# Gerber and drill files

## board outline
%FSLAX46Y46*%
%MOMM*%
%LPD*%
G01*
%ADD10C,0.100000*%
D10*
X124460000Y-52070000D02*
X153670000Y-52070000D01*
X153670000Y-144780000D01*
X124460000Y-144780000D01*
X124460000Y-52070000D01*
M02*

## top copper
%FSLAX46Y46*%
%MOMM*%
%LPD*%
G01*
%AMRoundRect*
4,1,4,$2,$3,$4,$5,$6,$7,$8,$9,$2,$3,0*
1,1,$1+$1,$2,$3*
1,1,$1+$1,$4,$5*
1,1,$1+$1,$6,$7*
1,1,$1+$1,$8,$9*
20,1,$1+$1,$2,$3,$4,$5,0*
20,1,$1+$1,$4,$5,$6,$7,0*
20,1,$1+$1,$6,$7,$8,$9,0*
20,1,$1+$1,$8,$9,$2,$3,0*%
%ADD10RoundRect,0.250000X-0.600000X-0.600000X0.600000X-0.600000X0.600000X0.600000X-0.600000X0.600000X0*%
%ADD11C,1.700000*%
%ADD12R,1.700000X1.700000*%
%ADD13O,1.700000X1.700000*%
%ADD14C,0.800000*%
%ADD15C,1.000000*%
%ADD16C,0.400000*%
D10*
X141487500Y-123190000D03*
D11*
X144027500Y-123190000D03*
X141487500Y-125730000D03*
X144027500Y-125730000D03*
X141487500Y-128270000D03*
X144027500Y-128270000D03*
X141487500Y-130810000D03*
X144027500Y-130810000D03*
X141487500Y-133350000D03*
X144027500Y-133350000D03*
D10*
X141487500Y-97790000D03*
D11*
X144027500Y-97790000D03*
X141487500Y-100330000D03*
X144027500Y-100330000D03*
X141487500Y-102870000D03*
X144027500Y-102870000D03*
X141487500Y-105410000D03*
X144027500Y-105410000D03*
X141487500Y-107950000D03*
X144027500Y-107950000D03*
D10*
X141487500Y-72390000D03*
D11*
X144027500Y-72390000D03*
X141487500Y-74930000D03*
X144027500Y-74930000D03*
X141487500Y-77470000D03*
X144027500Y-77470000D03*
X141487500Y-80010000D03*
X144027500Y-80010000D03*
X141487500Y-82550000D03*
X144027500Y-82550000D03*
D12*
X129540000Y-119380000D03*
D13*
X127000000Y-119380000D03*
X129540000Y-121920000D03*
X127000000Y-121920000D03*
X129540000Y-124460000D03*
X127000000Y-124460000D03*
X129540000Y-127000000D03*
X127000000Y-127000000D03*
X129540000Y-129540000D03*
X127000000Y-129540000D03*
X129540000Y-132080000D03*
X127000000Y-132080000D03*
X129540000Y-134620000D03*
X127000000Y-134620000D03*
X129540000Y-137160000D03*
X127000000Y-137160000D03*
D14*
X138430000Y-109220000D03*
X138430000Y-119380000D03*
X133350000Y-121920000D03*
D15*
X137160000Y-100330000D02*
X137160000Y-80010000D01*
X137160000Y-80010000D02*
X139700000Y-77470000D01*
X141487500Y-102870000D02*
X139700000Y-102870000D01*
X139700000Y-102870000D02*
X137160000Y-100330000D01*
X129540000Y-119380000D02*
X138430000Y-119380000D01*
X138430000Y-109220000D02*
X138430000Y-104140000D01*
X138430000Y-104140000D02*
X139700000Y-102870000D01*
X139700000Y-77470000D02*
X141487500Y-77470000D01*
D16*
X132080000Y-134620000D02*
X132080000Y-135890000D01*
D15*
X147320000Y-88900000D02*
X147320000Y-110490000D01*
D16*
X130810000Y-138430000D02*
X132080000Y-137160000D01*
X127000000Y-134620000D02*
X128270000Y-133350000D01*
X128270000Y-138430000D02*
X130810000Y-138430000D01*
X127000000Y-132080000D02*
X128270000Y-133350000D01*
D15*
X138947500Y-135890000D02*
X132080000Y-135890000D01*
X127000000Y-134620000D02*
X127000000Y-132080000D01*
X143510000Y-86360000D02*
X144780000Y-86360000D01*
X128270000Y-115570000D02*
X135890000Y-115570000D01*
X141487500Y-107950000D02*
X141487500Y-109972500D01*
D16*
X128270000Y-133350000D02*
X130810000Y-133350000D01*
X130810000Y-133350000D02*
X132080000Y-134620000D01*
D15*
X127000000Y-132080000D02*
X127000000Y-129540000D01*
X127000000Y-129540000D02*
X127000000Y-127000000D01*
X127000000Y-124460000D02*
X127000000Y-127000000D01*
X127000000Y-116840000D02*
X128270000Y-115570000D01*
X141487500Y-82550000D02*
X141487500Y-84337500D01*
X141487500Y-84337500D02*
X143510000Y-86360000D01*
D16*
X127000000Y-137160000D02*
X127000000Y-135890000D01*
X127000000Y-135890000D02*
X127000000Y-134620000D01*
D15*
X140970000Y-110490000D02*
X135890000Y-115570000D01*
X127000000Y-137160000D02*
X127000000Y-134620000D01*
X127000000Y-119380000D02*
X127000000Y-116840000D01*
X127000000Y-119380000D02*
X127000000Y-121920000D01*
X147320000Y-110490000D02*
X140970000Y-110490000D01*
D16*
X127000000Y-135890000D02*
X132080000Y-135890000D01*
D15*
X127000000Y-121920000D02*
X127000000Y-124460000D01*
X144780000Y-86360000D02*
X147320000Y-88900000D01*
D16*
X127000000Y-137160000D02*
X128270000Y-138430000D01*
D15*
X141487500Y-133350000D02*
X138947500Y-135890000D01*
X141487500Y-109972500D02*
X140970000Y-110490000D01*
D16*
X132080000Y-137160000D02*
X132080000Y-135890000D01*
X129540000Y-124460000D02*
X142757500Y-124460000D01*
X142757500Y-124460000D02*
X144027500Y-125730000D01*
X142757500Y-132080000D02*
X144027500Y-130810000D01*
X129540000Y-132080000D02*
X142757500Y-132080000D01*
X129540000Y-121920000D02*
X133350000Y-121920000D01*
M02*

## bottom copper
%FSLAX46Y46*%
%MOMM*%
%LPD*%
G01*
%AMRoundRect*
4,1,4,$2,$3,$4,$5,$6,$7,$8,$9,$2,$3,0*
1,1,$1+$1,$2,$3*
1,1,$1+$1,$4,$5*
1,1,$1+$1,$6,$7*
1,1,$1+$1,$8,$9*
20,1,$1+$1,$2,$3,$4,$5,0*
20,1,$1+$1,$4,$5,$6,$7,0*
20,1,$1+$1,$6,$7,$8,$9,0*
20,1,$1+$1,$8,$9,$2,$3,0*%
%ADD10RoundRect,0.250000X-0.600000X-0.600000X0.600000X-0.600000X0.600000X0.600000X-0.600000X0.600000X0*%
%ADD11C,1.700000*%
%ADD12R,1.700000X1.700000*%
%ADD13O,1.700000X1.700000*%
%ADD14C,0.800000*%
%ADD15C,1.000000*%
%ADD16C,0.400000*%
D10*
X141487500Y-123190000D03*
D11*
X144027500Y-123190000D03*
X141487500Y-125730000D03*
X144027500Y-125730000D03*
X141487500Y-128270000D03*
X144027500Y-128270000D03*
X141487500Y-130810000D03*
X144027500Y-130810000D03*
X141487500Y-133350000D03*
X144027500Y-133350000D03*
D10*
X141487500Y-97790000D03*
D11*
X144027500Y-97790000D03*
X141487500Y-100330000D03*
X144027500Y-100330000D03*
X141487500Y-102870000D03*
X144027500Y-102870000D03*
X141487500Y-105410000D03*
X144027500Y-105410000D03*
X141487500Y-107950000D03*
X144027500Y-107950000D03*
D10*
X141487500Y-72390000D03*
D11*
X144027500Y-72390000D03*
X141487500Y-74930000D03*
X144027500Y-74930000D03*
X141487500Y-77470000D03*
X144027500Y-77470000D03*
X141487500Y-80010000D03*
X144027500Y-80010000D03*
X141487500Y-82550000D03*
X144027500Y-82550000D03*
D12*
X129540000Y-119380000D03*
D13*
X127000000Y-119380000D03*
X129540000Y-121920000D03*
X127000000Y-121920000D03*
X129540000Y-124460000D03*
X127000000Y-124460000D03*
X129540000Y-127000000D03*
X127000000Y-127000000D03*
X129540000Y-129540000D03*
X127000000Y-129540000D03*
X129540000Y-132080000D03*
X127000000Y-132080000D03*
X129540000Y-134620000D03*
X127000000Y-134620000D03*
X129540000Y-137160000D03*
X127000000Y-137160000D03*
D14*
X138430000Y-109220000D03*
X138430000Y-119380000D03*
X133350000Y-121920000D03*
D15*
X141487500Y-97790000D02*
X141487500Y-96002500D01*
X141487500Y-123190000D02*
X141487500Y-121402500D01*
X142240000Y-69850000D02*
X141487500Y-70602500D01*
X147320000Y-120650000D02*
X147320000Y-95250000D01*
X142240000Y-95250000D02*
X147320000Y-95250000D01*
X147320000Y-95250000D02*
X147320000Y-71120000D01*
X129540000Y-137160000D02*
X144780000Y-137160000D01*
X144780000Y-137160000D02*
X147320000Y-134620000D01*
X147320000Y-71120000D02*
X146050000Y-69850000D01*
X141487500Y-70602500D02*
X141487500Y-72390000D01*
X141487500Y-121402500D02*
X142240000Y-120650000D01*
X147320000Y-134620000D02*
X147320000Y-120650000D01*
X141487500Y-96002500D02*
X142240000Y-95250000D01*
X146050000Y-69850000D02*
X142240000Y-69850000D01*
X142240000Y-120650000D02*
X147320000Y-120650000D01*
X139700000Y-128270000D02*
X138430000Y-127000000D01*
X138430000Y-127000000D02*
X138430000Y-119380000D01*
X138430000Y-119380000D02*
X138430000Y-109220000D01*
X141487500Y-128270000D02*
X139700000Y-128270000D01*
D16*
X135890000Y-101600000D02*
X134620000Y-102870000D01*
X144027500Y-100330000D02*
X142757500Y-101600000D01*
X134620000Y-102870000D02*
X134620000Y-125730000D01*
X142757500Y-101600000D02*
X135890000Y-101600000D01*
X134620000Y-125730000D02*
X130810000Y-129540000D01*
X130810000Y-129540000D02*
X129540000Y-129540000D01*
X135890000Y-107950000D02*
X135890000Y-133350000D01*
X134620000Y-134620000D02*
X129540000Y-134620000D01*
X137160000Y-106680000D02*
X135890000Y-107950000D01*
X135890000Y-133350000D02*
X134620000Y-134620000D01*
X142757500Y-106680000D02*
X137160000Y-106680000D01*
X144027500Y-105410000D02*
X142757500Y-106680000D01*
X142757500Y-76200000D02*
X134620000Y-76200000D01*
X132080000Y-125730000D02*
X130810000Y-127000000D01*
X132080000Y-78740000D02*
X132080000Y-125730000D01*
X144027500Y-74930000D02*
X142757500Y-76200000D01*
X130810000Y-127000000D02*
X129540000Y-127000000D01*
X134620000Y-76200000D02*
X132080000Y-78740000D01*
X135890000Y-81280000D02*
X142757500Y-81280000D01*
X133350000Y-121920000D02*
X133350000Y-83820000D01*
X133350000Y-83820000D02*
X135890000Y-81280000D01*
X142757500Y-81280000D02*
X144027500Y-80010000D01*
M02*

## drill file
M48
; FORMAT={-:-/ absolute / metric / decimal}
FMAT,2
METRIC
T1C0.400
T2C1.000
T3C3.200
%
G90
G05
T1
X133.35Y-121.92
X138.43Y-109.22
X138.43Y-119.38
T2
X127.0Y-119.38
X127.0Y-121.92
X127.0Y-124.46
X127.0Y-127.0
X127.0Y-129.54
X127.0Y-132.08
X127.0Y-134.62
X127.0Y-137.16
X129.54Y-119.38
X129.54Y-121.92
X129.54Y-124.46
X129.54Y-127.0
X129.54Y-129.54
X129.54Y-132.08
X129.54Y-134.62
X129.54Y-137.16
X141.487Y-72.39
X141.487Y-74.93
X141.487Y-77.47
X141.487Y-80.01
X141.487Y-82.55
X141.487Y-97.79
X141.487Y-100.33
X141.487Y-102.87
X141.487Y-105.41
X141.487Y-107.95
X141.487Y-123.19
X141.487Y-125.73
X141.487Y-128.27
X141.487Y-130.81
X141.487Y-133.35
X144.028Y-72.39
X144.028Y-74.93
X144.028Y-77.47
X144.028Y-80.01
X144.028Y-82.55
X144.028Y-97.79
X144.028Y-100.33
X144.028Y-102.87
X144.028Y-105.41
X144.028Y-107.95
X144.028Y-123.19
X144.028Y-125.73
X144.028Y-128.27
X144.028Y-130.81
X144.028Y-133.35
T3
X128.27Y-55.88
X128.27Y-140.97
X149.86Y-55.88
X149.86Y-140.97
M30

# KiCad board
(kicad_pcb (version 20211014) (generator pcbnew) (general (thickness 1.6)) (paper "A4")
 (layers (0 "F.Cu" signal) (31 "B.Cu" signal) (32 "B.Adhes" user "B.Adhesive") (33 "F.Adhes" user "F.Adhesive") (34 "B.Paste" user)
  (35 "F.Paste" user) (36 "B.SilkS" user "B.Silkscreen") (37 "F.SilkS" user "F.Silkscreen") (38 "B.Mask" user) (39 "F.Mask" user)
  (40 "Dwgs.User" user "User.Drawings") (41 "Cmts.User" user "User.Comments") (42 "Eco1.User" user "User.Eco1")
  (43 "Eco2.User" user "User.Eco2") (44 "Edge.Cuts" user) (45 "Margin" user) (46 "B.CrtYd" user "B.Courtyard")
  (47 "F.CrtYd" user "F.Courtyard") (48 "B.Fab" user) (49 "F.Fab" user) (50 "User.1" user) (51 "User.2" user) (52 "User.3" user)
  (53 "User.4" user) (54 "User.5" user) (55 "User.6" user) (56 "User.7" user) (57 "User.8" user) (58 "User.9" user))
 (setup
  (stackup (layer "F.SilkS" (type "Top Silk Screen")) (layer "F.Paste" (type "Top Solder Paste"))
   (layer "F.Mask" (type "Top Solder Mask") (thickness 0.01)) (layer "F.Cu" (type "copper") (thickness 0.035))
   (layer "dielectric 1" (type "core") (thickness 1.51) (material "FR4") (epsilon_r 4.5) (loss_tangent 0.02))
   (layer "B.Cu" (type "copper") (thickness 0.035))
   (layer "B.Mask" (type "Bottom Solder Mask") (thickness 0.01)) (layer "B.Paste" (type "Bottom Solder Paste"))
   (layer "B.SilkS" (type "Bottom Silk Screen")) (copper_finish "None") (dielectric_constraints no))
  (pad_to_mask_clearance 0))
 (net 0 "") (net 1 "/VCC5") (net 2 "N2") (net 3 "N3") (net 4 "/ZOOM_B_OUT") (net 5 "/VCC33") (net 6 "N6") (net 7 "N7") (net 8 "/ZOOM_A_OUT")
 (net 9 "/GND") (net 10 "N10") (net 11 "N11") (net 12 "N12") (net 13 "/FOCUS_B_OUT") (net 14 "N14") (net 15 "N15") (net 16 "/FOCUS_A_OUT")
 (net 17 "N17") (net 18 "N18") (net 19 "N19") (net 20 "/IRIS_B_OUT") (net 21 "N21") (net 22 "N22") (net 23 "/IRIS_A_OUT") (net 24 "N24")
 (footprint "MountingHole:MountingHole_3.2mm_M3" (layer "F.Cu") (at 149.86 55.88)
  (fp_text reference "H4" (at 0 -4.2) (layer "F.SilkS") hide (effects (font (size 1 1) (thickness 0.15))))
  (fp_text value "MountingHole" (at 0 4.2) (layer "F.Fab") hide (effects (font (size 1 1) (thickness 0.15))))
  (pad "" np_thru_hole circle locked (at 0 0) (size 3.2 3.2) (drill 3.2) (layers *.Cu *.Mask)))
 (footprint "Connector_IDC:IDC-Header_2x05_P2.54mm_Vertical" (layer "F.Cu") (at 141.4875 123.19)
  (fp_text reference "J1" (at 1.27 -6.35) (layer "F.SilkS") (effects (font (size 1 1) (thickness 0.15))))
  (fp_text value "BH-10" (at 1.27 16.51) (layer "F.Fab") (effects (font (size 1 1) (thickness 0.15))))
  (pad "1" thru_hole roundrect locked (at 0 0) (size 1.7 1.7) (drill 1) (layers *.Cu *.Mask) (roundrect_rratio 0.1470588235) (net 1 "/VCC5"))
  (pad "2" thru_hole circle locked (at 2.54 0) (size 1.7 1.7) (drill 1) (layers *.Cu *.Mask) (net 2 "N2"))
  (pad "3" thru_hole circle locked (at 0 2.54) (size 1.7 1.7) (drill 1) (layers *.Cu *.Mask) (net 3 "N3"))
  (pad "4" thru_hole circle locked (at 2.54 2.54) (size 1.7 1.7) (drill 1) (layers *.Cu *.Mask) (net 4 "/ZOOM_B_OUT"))
  (pad "5" thru_hole circle locked (at 0 5.08) (size 1.7 1.7) (drill 1) (layers *.Cu *.Mask) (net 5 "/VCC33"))
  (pad "6" thru_hole circle locked (at 2.54 5.08) (size 1.7 1.7) (drill 1) (layers *.Cu *.Mask) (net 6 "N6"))
  (pad "7" thru_hole circle locked (at 0 7.62) (size 1.7 1.7) (drill 1) (layers *.Cu *.Mask) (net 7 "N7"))
  (pad "8" thru_hole circle locked (at 2.54 7.62) (size 1.7 1.7) (drill 1) (layers *.Cu *.Mask) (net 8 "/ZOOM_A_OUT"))
  (pad "9" thru_hole circle locked (at 0 10.16) (size 1.7 1.7) (drill 1) (layers *.Cu *.Mask) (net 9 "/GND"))
  (pad "10" thru_hole circle locked (at 2.54 10.16) (size 1.7 1.7) (drill 1) (layers *.Cu *.Mask) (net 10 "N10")))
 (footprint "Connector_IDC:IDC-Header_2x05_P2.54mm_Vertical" (layer "F.Cu") (at 141.4875 97.79)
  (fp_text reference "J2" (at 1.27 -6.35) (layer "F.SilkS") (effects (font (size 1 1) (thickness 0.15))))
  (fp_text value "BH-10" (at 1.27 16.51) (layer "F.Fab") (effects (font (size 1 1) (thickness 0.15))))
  (pad "1" thru_hole roundrect locked (at 0 0) (size 1.7 1.7) (drill 1) (layers *.Cu *.Mask) (roundrect_rratio 0.1470588235) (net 1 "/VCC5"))
  (pad "2" thru_hole circle locked (at 2.54 0) (size 1.7 1.7) (drill 1) (layers *.Cu *.Mask) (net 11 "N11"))
  (pad "3" thru_hole circle locked (at 0 2.54) (size 1.7 1.7) (drill 1) (layers *.Cu *.Mask) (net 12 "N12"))
  (pad "4" thru_hole circle locked (at 2.54 2.54) (size 1.7 1.7) (drill 1) (layers *.Cu *.Mask) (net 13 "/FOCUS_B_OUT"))
  (pad "5" thru_hole circle locked (at 0 5.08) (size 1.7 1.7) (drill 1) (layers *.Cu *.Mask) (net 5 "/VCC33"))
  (pad "6" thru_hole circle locked (at 2.54 5.08) (size 1.7 1.7) (drill 1) (layers *.Cu *.Mask) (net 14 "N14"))
  (pad "7" thru_hole circle locked (at 0 7.62) (size 1.7 1.7) (drill 1) (layers *.Cu *.Mask) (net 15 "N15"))
  (pad "8" thru_hole circle locked (at 2.54 7.62) (size 1.7 1.7) (drill 1) (layers *.Cu *.Mask) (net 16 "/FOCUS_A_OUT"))
  (pad "9" thru_hole circle locked (at 0 10.16) (size 1.7 1.7) (drill 1) (layers *.Cu *.Mask) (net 9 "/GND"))
  (pad "10" thru_hole circle locked (at 2.54 10.16) (size 1.7 1.7) (drill 1) (layers *.Cu *.Mask) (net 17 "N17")))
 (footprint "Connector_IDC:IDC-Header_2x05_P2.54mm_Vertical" (layer "F.Cu") (at 141.4875 72.39)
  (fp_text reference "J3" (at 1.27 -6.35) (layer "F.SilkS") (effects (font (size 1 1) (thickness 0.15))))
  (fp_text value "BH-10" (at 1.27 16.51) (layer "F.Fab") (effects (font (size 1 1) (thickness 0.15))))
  (pad "1" thru_hole roundrect locked (at 0 0) (size 1.7 1.7) (drill 1) (layers *.Cu *.Mask) (roundrect_rratio 0.1470588235) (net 1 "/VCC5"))
  (pad "2" thru_hole circle locked (at 2.54 0) (size 1.7 1.7) (drill 1) (layers *.Cu *.Mask) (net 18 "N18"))
  (pad "3" thru_hole circle locked (at 0 2.54) (size 1.7 1.7) (drill 1) (layers *.Cu *.Mask) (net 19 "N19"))
  (pad "4" thru_hole circle locked (at 2.54 2.54) (size 1.7 1.7) (drill 1) (layers *.Cu *.Mask) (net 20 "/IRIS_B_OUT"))
  (pad "5" thru_hole circle locked (at 0 5.08) (size 1.7 1.7) (drill 1) (layers *.Cu *.Mask) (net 5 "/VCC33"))
  (pad "6" thru_hole circle locked (at 2.54 5.08) (size 1.7 1.7) (drill 1) (layers *.Cu *.Mask) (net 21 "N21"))
  (pad "7" thru_hole circle locked (at 0 7.62) (size 1.7 1.7) (drill 1) (layers *.Cu *.Mask) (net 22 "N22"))
  (pad "8" thru_hole circle locked (at 2.54 7.62) (size 1.7 1.7) (drill 1) (layers *.Cu *.Mask) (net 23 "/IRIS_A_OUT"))
  (pad "9" thru_hole circle locked (at 0 10.16) (size 1.7 1.7) (drill 1) (layers *.Cu *.Mask) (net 9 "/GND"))
  (pad "10" thru_hole circle locked (at 2.54 10.16) (size 1.7 1.7) (drill 1) (layers *.Cu *.Mask) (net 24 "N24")))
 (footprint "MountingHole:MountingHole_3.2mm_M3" (layer "F.Cu") (at 128.27 140.97)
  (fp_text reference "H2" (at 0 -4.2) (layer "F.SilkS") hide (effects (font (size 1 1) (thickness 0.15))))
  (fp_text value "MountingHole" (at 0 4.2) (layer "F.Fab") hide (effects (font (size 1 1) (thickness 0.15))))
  (pad "" np_thru_hole circle locked (at 0 0) (size 3.2 3.2) (drill 3.2) (layers *.Cu *.Mask)))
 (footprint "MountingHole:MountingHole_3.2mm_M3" (layer "F.Cu") (at 149.86 140.97)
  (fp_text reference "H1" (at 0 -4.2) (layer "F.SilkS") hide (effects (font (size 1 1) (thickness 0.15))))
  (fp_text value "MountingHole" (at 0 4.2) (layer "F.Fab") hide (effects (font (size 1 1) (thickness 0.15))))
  (pad "" np_thru_hole circle locked (at 0 0) (size 3.2 3.2) (drill 3.2) (layers *.Cu *.Mask)))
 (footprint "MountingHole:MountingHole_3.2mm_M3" (layer "F.Cu") (at 128.27 55.88)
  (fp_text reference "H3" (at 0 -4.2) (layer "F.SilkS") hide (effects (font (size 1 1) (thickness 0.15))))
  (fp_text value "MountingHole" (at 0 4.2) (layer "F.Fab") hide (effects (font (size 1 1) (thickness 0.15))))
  (pad "" np_thru_hole circle locked (at 0 0) (size 3.2 3.2) (drill 3.2) (layers *.Cu *.Mask)))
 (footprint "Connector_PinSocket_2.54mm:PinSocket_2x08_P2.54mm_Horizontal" (layer "F.Cu") (at 129.54 119.38)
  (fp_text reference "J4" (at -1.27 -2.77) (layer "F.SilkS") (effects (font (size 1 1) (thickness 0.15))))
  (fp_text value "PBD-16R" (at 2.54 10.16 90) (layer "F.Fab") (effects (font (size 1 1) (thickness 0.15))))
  (pad "1" thru_hole rect locked (at 0 0) (size 1.7 1.7) (drill 1) (layers *.Cu *.Mask) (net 5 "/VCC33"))
  (pad "2" thru_hole oval locked (at -2.54 0) (size 1.7 1.7) (drill 1) (layers *.Cu *.Mask) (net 9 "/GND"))
  (pad "3" thru_hole oval locked (at 0 2.54) (size 1.7 1.7) (drill 1) (layers *.Cu *.Mask) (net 23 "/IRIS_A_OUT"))
  (pad "4" thru_hole oval locked (at -2.54 2.54) (size 1.7 1.7) (drill 1) (layers *.Cu *.Mask) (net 9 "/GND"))
  (pad "5" thru_hole oval locked (at 0 5.08) (size 1.7 1.7) (drill 1) (layers *.Cu *.Mask) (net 4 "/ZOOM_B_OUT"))
  (pad "6" thru_hole oval locked (at -2.54 5.08) (size 1.7 1.7) (drill 1) (layers *.Cu *.Mask) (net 9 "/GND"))
  (pad "7" thru_hole oval locked (at 0 7.62) (size 1.7 1.7) (drill 1) (layers *.Cu *.Mask) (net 20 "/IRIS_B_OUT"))
  (pad "8" thru_hole oval locked (at -2.54 7.62) (size 1.7 1.7) (drill 1) (layers *.Cu *.Mask) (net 9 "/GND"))
  (pad "9" thru_hole oval locked (at 0 10.16) (size 1.7 1.7) (drill 1) (layers *.Cu *.Mask) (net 13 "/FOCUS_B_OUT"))
  (pad "10" thru_hole oval locked (at -2.54 10.16) (size 1.7 1.7) (drill 1) (layers *.Cu *.Mask) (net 9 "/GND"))
  (pad "11" thru_hole oval locked (at 0 12.7) (size 1.7 1.7) (drill 1) (layers *.Cu *.Mask) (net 8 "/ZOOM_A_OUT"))
  (pad "12" thru_hole oval locked (at -2.54 12.7) (size 1.7 1.7) (drill 1) (layers *.Cu *.Mask) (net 9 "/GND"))
  (pad "13" thru_hole oval locked (at 0 15.24) (size 1.7 1.7) (drill 1) (layers *.Cu *.Mask) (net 16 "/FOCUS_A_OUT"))
  (pad "14" thru_hole oval locked (at -2.54 15.24) (size 1.7 1.7) (drill 1) (layers *.Cu *.Mask) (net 9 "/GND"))
  (pad "15" thru_hole oval locked (at 0 17.78) (size 1.7 1.7) (drill 1) (layers *.Cu *.Mask) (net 1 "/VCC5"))
  (pad "16" thru_hole oval locked (at -2.54 17.78) (size 1.7 1.7) (drill 1) (layers *.Cu *.Mask) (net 9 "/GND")))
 (gr_rect (start 124.46 52.07) (end 153.67 144.78) (layer "Edge.Cuts") (width 0.1) (fill none))
 (segment (start 141.4875 97.79) (end 141.4875 96.0025) (width 1) (layer "B.Cu") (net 1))
 (segment (start 141.4875 123.19) (end 141.4875 121.4025) (width 1) (layer "B.Cu") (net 1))
 (segment (start 142.24 69.85) (end 141.4875 70.6025) (width 1) (layer "B.Cu") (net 1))
 (segment (start 147.32 120.65) (end 147.32 95.25) (width 1) (layer "B.Cu") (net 1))
 (segment (start 142.24 95.25) (end 147.32 95.25) (width 1) (layer "B.Cu") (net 1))
 (segment (start 147.32 95.25) (end 147.32 71.12) (width 1) (layer "B.Cu") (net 1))
 (segment (start 129.54 137.16) (end 144.78 137.16) (width 1) (layer "B.Cu") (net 1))
 (segment (start 144.78 137.16) (end 147.32 134.62) (width 1) (layer "B.Cu") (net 1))
 (segment (start 147.32 71.12) (end 146.05 69.85) (width 1) (layer "B.Cu") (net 1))
 (segment (start 141.4875 70.6025) (end 141.4875 72.39) (width 1) (layer "B.Cu") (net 1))
 (segment (start 141.4875 121.4025) (end 142.24 120.65) (width 1) (layer "B.Cu") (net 1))
 (segment (start 147.32 134.62) (end 147.32 120.65) (width 1) (layer "B.Cu") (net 1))
 (segment (start 141.4875 96.0025) (end 142.24 95.25) (width 1) (layer "B.Cu") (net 1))
 (segment (start 146.05 69.85) (end 142.24 69.85) (width 1) (layer "B.Cu") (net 1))
 (segment (start 142.24 120.65) (end 147.32 120.65) (width 1) (layer "B.Cu") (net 1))
 (segment (start 137.16 100.33) (end 137.16 80.01) (width 1) (layer "F.Cu") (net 5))
 (segment (start 137.16 80.01) (end 139.7 77.47) (width 1) (layer "F.Cu") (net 5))
 (segment (start 141.4875 102.87) (end 139.7 102.87) (width 1) (layer "F.Cu") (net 5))
 (segment (start 139.7 102.87) (end 137.16 100.33) (width 1) (layer "F.Cu") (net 5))
 (segment (start 129.54 119.38) (end 138.43 119.38) (width 1) (layer "F.Cu") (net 5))
 (segment (start 138.43 109.22) (end 138.43 104.14) (width 1) (layer "F.Cu") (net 5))
 (segment (start 138.43 104.14) (end 139.7 102.87) (width 1) (layer "F.Cu") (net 5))
 (segment (start 139.7 77.47) (end 141.4875 77.47) (width 1) (layer "F.Cu") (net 5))
 (via (at 138.43 109.22) (size 0.8) (drill 0.4) (layers "F.Cu" "B.Cu") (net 5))
 (via (at 138.43 119.38) (size 0.8) (drill 0.4) (layers "F.Cu" "B.Cu") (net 5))
 (segment (start 139.7 128.27) (end 138.43 127) (width 1) (layer "B.Cu") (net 5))
 (segment (start 138.43 127) (end 138.43 119.38) (width 1) (layer "B.Cu") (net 5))
 (segment (start 138.43 119.38) (end 138.43 109.22) (width 1) (layer "B.Cu") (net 5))
 (segment (start 141.4875 128.27) (end 139.7 128.27) (width 1) (layer "B.Cu") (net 5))
 (segment (start 132.08 134.62) (end 132.08 135.89) (width 0.4) (layer "F.Cu") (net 9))
 (segment (start 147.32 88.9) (end 147.32 110.49) (width 1) (layer "F.Cu") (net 9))
 (segment (start 130.81 138.43) (end 132.08 137.16) (width 0.4) (layer "F.Cu") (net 9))
 (segment (start 127 134.62) (end 128.27 133.35) (width 0.4) (layer "F.Cu") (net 9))
 (segment (start 128.27 138.43) (end 130.81 138.43) (width 0.4) (layer "F.Cu") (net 9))
 (segment (start 127 132.08) (end 128.27 133.35) (width 0.4) (layer "F.Cu") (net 9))
 (segment (start 138.9475 135.89) (end 132.08 135.89) (width 1) (layer "F.Cu") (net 9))
 (segment (start 127 134.62) (end 127 132.08) (width 1) (layer "F.Cu") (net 9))
 (segment (start 143.51 86.36) (end 144.78 86.36) (width 1) (layer "F.Cu") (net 9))
 (segment (start 128.27 115.57) (end 135.89 115.57) (width 1) (layer "F.Cu") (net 9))
 (segment (start 141.4875 107.95) (end 141.4875 109.9725) (width 1) (layer "F.Cu") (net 9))
 (segment (start 128.27 133.35) (end 130.81 133.35) (width 0.4) (layer "F.Cu") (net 9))
 (segment (start 130.81 133.35) (end 132.08 134.62) (width 0.4) (layer "F.Cu") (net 9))
 (segment (start 127 132.08) (end 127 129.54) (width 1) (layer "F.Cu") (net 9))
 (segment (start 127 129.54) (end 127 127) (width 1) (layer "F.Cu") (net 9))
 (segment (start 127 124.46) (end 127 127) (width 1) (layer "F.Cu") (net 9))
 (segment (start 127 116.84) (end 128.27 115.57) (width 1) (layer "F.Cu") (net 9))
 (segment (start 141.4875 82.55) (end 141.4875 84.3375) (width 1) (layer "F.Cu") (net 9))
 (segment (start 141.4875 84.3375) (end 143.51 86.36) (width 1) (layer "F.Cu") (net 9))
 (segment (start 127 137.16) (end 127 135.89) (width 0.4) (layer "F.Cu") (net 9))
 (segment (start 127 135.89) (end 127 134.62) (width 0.4) (layer "F.Cu") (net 9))
 (segment (start 140.97 110.49) (end 135.89 115.57) (width 1) (layer "F.Cu") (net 9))
 (segment (start 127 137.16) (end 127 134.62) (width 1) (layer "F.Cu") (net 9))
 (segment (start 127 119.38) (end 127 116.84) (width 1) (layer "F.Cu") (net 9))
 (segment (start 127 119.38) (end 127 121.92) (width 1) (layer "F.Cu") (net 9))
 (segment (start 147.32 110.49) (end 140.97 110.49) (width 1) (layer "F.Cu") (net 9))
 (segment (start 127 135.89) (end 132.08 135.89) (width 0.4) (layer "F.Cu") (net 9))
 (segment (start 127 121.92) (end 127 124.46) (width 1) (layer "F.Cu") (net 9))
 (segment (start 144.78 86.36) (end 147.32 88.9) (width 1) (layer "F.Cu") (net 9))
 (segment (start 127 137.16) (end 128.27 138.43) (width 0.4) (layer "F.Cu") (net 9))
 (segment (start 141.4875 133.35) (end 138.9475 135.89) (width 1) (layer "F.Cu") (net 9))
 (segment (start 141.4875 109.9725) (end 140.97 110.49) (width 1) (layer "F.Cu") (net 9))
 (segment (start 132.08 137.16) (end 132.08 135.89) (width 0.4) (layer "F.Cu") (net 9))
 (segment (start 129.54 124.46) (end 142.7575 124.46) (width 0.4) (layer "F.Cu") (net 4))
 (segment (start 142.7575 124.46) (end 144.0275 125.73) (width 0.4) (layer "F.Cu") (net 4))
 (segment (start 142.7575 132.08) (end 144.0275 130.81) (width 0.4) (layer "F.Cu") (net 8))
 (segment (start 129.54 132.08) (end 142.7575 132.08) (width 0.4) (layer "F.Cu") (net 8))
 (segment (start 135.89 101.6) (end 134.62 102.87) (width 0.4) (layer "B.Cu") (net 13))
 (segment (start 144.0275 100.33) (end 142.7575 101.6) (width 0.4) (layer "B.Cu") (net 13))
 (segment (start 134.62 102.87) (end 134.62 125.73) (width 0.4) (layer "B.Cu") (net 13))
 (segment (start 142.7575 101.6) (end 135.89 101.6) (width 0.4) (layer "B.Cu") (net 13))
 (segment (start 134.62 125.73) (end 130.81 129.54) (width 0.4) (layer "B.Cu") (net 13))
 (segment (start 130.81 129.54) (end 129.54 129.54) (width 0.4) (layer "B.Cu") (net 13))
 (segment (start 135.89 107.95) (end 135.89 133.35) (width 0.4) (layer "B.Cu") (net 16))
 (segment (start 134.62 134.62) (end 129.54 134.62) (width 0.4) (layer "B.Cu") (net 16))
 (segment (start 137.16 106.68) (end 135.89 107.95) (width 0.4) (layer "B.Cu") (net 16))
 (segment (start 135.89 133.35) (end 134.62 134.62) (width 0.4) (layer "B.Cu") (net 16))
 (segment (start 142.7575 106.68) (end 137.16 106.68) (width 0.4) (layer "B.Cu") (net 16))
 (segment (start 144.0275 105.41) (end 142.7575 106.68) (width 0.4) (layer "B.Cu") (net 16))
 (segment (start 142.7575 76.2) (end 134.62 76.2) (width 0.4) (layer "B.Cu") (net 20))
 (segment (start 132.08 125.73) (end 130.81 127) (width 0.4) (layer "B.Cu") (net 20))
 (segment (start 132.08 78.74) (end 132.08 125.73) (width 0.4) (layer "B.Cu") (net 20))
 (segment (start 144.0275 74.93) (end 142.7575 76.2) (width 0.4) (layer "B.Cu") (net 20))
 (segment (start 130.81 127) (end 129.54 127) (width 0.4) (layer "B.Cu") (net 20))
 (segment (start 134.62 76.2) (end 132.08 78.74) (width 0.4) (layer "B.Cu") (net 20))
 (segment (start 129.54 121.92) (end 133.35 121.92) (width 0.4) (layer "F.Cu") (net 23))
 (via (at 133.35 121.92) (size 0.8) (drill 0.4) (layers "F.Cu" "B.Cu") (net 23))
 (segment (start 135.89 81.28) (end 142.7575 81.28) (width 0.4) (layer "B.Cu") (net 23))
 (segment (start 133.35 121.92) (end 133.35 83.82) (width 0.4) (layer "B.Cu") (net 23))
 (segment (start 133.35 83.82) (end 135.89 81.28) (width 0.4) (layer "B.Cu") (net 23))
 (segment (start 142.7575 81.28) (end 144.0275 80.01) (width 0.4) (layer "B.Cu") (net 23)))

